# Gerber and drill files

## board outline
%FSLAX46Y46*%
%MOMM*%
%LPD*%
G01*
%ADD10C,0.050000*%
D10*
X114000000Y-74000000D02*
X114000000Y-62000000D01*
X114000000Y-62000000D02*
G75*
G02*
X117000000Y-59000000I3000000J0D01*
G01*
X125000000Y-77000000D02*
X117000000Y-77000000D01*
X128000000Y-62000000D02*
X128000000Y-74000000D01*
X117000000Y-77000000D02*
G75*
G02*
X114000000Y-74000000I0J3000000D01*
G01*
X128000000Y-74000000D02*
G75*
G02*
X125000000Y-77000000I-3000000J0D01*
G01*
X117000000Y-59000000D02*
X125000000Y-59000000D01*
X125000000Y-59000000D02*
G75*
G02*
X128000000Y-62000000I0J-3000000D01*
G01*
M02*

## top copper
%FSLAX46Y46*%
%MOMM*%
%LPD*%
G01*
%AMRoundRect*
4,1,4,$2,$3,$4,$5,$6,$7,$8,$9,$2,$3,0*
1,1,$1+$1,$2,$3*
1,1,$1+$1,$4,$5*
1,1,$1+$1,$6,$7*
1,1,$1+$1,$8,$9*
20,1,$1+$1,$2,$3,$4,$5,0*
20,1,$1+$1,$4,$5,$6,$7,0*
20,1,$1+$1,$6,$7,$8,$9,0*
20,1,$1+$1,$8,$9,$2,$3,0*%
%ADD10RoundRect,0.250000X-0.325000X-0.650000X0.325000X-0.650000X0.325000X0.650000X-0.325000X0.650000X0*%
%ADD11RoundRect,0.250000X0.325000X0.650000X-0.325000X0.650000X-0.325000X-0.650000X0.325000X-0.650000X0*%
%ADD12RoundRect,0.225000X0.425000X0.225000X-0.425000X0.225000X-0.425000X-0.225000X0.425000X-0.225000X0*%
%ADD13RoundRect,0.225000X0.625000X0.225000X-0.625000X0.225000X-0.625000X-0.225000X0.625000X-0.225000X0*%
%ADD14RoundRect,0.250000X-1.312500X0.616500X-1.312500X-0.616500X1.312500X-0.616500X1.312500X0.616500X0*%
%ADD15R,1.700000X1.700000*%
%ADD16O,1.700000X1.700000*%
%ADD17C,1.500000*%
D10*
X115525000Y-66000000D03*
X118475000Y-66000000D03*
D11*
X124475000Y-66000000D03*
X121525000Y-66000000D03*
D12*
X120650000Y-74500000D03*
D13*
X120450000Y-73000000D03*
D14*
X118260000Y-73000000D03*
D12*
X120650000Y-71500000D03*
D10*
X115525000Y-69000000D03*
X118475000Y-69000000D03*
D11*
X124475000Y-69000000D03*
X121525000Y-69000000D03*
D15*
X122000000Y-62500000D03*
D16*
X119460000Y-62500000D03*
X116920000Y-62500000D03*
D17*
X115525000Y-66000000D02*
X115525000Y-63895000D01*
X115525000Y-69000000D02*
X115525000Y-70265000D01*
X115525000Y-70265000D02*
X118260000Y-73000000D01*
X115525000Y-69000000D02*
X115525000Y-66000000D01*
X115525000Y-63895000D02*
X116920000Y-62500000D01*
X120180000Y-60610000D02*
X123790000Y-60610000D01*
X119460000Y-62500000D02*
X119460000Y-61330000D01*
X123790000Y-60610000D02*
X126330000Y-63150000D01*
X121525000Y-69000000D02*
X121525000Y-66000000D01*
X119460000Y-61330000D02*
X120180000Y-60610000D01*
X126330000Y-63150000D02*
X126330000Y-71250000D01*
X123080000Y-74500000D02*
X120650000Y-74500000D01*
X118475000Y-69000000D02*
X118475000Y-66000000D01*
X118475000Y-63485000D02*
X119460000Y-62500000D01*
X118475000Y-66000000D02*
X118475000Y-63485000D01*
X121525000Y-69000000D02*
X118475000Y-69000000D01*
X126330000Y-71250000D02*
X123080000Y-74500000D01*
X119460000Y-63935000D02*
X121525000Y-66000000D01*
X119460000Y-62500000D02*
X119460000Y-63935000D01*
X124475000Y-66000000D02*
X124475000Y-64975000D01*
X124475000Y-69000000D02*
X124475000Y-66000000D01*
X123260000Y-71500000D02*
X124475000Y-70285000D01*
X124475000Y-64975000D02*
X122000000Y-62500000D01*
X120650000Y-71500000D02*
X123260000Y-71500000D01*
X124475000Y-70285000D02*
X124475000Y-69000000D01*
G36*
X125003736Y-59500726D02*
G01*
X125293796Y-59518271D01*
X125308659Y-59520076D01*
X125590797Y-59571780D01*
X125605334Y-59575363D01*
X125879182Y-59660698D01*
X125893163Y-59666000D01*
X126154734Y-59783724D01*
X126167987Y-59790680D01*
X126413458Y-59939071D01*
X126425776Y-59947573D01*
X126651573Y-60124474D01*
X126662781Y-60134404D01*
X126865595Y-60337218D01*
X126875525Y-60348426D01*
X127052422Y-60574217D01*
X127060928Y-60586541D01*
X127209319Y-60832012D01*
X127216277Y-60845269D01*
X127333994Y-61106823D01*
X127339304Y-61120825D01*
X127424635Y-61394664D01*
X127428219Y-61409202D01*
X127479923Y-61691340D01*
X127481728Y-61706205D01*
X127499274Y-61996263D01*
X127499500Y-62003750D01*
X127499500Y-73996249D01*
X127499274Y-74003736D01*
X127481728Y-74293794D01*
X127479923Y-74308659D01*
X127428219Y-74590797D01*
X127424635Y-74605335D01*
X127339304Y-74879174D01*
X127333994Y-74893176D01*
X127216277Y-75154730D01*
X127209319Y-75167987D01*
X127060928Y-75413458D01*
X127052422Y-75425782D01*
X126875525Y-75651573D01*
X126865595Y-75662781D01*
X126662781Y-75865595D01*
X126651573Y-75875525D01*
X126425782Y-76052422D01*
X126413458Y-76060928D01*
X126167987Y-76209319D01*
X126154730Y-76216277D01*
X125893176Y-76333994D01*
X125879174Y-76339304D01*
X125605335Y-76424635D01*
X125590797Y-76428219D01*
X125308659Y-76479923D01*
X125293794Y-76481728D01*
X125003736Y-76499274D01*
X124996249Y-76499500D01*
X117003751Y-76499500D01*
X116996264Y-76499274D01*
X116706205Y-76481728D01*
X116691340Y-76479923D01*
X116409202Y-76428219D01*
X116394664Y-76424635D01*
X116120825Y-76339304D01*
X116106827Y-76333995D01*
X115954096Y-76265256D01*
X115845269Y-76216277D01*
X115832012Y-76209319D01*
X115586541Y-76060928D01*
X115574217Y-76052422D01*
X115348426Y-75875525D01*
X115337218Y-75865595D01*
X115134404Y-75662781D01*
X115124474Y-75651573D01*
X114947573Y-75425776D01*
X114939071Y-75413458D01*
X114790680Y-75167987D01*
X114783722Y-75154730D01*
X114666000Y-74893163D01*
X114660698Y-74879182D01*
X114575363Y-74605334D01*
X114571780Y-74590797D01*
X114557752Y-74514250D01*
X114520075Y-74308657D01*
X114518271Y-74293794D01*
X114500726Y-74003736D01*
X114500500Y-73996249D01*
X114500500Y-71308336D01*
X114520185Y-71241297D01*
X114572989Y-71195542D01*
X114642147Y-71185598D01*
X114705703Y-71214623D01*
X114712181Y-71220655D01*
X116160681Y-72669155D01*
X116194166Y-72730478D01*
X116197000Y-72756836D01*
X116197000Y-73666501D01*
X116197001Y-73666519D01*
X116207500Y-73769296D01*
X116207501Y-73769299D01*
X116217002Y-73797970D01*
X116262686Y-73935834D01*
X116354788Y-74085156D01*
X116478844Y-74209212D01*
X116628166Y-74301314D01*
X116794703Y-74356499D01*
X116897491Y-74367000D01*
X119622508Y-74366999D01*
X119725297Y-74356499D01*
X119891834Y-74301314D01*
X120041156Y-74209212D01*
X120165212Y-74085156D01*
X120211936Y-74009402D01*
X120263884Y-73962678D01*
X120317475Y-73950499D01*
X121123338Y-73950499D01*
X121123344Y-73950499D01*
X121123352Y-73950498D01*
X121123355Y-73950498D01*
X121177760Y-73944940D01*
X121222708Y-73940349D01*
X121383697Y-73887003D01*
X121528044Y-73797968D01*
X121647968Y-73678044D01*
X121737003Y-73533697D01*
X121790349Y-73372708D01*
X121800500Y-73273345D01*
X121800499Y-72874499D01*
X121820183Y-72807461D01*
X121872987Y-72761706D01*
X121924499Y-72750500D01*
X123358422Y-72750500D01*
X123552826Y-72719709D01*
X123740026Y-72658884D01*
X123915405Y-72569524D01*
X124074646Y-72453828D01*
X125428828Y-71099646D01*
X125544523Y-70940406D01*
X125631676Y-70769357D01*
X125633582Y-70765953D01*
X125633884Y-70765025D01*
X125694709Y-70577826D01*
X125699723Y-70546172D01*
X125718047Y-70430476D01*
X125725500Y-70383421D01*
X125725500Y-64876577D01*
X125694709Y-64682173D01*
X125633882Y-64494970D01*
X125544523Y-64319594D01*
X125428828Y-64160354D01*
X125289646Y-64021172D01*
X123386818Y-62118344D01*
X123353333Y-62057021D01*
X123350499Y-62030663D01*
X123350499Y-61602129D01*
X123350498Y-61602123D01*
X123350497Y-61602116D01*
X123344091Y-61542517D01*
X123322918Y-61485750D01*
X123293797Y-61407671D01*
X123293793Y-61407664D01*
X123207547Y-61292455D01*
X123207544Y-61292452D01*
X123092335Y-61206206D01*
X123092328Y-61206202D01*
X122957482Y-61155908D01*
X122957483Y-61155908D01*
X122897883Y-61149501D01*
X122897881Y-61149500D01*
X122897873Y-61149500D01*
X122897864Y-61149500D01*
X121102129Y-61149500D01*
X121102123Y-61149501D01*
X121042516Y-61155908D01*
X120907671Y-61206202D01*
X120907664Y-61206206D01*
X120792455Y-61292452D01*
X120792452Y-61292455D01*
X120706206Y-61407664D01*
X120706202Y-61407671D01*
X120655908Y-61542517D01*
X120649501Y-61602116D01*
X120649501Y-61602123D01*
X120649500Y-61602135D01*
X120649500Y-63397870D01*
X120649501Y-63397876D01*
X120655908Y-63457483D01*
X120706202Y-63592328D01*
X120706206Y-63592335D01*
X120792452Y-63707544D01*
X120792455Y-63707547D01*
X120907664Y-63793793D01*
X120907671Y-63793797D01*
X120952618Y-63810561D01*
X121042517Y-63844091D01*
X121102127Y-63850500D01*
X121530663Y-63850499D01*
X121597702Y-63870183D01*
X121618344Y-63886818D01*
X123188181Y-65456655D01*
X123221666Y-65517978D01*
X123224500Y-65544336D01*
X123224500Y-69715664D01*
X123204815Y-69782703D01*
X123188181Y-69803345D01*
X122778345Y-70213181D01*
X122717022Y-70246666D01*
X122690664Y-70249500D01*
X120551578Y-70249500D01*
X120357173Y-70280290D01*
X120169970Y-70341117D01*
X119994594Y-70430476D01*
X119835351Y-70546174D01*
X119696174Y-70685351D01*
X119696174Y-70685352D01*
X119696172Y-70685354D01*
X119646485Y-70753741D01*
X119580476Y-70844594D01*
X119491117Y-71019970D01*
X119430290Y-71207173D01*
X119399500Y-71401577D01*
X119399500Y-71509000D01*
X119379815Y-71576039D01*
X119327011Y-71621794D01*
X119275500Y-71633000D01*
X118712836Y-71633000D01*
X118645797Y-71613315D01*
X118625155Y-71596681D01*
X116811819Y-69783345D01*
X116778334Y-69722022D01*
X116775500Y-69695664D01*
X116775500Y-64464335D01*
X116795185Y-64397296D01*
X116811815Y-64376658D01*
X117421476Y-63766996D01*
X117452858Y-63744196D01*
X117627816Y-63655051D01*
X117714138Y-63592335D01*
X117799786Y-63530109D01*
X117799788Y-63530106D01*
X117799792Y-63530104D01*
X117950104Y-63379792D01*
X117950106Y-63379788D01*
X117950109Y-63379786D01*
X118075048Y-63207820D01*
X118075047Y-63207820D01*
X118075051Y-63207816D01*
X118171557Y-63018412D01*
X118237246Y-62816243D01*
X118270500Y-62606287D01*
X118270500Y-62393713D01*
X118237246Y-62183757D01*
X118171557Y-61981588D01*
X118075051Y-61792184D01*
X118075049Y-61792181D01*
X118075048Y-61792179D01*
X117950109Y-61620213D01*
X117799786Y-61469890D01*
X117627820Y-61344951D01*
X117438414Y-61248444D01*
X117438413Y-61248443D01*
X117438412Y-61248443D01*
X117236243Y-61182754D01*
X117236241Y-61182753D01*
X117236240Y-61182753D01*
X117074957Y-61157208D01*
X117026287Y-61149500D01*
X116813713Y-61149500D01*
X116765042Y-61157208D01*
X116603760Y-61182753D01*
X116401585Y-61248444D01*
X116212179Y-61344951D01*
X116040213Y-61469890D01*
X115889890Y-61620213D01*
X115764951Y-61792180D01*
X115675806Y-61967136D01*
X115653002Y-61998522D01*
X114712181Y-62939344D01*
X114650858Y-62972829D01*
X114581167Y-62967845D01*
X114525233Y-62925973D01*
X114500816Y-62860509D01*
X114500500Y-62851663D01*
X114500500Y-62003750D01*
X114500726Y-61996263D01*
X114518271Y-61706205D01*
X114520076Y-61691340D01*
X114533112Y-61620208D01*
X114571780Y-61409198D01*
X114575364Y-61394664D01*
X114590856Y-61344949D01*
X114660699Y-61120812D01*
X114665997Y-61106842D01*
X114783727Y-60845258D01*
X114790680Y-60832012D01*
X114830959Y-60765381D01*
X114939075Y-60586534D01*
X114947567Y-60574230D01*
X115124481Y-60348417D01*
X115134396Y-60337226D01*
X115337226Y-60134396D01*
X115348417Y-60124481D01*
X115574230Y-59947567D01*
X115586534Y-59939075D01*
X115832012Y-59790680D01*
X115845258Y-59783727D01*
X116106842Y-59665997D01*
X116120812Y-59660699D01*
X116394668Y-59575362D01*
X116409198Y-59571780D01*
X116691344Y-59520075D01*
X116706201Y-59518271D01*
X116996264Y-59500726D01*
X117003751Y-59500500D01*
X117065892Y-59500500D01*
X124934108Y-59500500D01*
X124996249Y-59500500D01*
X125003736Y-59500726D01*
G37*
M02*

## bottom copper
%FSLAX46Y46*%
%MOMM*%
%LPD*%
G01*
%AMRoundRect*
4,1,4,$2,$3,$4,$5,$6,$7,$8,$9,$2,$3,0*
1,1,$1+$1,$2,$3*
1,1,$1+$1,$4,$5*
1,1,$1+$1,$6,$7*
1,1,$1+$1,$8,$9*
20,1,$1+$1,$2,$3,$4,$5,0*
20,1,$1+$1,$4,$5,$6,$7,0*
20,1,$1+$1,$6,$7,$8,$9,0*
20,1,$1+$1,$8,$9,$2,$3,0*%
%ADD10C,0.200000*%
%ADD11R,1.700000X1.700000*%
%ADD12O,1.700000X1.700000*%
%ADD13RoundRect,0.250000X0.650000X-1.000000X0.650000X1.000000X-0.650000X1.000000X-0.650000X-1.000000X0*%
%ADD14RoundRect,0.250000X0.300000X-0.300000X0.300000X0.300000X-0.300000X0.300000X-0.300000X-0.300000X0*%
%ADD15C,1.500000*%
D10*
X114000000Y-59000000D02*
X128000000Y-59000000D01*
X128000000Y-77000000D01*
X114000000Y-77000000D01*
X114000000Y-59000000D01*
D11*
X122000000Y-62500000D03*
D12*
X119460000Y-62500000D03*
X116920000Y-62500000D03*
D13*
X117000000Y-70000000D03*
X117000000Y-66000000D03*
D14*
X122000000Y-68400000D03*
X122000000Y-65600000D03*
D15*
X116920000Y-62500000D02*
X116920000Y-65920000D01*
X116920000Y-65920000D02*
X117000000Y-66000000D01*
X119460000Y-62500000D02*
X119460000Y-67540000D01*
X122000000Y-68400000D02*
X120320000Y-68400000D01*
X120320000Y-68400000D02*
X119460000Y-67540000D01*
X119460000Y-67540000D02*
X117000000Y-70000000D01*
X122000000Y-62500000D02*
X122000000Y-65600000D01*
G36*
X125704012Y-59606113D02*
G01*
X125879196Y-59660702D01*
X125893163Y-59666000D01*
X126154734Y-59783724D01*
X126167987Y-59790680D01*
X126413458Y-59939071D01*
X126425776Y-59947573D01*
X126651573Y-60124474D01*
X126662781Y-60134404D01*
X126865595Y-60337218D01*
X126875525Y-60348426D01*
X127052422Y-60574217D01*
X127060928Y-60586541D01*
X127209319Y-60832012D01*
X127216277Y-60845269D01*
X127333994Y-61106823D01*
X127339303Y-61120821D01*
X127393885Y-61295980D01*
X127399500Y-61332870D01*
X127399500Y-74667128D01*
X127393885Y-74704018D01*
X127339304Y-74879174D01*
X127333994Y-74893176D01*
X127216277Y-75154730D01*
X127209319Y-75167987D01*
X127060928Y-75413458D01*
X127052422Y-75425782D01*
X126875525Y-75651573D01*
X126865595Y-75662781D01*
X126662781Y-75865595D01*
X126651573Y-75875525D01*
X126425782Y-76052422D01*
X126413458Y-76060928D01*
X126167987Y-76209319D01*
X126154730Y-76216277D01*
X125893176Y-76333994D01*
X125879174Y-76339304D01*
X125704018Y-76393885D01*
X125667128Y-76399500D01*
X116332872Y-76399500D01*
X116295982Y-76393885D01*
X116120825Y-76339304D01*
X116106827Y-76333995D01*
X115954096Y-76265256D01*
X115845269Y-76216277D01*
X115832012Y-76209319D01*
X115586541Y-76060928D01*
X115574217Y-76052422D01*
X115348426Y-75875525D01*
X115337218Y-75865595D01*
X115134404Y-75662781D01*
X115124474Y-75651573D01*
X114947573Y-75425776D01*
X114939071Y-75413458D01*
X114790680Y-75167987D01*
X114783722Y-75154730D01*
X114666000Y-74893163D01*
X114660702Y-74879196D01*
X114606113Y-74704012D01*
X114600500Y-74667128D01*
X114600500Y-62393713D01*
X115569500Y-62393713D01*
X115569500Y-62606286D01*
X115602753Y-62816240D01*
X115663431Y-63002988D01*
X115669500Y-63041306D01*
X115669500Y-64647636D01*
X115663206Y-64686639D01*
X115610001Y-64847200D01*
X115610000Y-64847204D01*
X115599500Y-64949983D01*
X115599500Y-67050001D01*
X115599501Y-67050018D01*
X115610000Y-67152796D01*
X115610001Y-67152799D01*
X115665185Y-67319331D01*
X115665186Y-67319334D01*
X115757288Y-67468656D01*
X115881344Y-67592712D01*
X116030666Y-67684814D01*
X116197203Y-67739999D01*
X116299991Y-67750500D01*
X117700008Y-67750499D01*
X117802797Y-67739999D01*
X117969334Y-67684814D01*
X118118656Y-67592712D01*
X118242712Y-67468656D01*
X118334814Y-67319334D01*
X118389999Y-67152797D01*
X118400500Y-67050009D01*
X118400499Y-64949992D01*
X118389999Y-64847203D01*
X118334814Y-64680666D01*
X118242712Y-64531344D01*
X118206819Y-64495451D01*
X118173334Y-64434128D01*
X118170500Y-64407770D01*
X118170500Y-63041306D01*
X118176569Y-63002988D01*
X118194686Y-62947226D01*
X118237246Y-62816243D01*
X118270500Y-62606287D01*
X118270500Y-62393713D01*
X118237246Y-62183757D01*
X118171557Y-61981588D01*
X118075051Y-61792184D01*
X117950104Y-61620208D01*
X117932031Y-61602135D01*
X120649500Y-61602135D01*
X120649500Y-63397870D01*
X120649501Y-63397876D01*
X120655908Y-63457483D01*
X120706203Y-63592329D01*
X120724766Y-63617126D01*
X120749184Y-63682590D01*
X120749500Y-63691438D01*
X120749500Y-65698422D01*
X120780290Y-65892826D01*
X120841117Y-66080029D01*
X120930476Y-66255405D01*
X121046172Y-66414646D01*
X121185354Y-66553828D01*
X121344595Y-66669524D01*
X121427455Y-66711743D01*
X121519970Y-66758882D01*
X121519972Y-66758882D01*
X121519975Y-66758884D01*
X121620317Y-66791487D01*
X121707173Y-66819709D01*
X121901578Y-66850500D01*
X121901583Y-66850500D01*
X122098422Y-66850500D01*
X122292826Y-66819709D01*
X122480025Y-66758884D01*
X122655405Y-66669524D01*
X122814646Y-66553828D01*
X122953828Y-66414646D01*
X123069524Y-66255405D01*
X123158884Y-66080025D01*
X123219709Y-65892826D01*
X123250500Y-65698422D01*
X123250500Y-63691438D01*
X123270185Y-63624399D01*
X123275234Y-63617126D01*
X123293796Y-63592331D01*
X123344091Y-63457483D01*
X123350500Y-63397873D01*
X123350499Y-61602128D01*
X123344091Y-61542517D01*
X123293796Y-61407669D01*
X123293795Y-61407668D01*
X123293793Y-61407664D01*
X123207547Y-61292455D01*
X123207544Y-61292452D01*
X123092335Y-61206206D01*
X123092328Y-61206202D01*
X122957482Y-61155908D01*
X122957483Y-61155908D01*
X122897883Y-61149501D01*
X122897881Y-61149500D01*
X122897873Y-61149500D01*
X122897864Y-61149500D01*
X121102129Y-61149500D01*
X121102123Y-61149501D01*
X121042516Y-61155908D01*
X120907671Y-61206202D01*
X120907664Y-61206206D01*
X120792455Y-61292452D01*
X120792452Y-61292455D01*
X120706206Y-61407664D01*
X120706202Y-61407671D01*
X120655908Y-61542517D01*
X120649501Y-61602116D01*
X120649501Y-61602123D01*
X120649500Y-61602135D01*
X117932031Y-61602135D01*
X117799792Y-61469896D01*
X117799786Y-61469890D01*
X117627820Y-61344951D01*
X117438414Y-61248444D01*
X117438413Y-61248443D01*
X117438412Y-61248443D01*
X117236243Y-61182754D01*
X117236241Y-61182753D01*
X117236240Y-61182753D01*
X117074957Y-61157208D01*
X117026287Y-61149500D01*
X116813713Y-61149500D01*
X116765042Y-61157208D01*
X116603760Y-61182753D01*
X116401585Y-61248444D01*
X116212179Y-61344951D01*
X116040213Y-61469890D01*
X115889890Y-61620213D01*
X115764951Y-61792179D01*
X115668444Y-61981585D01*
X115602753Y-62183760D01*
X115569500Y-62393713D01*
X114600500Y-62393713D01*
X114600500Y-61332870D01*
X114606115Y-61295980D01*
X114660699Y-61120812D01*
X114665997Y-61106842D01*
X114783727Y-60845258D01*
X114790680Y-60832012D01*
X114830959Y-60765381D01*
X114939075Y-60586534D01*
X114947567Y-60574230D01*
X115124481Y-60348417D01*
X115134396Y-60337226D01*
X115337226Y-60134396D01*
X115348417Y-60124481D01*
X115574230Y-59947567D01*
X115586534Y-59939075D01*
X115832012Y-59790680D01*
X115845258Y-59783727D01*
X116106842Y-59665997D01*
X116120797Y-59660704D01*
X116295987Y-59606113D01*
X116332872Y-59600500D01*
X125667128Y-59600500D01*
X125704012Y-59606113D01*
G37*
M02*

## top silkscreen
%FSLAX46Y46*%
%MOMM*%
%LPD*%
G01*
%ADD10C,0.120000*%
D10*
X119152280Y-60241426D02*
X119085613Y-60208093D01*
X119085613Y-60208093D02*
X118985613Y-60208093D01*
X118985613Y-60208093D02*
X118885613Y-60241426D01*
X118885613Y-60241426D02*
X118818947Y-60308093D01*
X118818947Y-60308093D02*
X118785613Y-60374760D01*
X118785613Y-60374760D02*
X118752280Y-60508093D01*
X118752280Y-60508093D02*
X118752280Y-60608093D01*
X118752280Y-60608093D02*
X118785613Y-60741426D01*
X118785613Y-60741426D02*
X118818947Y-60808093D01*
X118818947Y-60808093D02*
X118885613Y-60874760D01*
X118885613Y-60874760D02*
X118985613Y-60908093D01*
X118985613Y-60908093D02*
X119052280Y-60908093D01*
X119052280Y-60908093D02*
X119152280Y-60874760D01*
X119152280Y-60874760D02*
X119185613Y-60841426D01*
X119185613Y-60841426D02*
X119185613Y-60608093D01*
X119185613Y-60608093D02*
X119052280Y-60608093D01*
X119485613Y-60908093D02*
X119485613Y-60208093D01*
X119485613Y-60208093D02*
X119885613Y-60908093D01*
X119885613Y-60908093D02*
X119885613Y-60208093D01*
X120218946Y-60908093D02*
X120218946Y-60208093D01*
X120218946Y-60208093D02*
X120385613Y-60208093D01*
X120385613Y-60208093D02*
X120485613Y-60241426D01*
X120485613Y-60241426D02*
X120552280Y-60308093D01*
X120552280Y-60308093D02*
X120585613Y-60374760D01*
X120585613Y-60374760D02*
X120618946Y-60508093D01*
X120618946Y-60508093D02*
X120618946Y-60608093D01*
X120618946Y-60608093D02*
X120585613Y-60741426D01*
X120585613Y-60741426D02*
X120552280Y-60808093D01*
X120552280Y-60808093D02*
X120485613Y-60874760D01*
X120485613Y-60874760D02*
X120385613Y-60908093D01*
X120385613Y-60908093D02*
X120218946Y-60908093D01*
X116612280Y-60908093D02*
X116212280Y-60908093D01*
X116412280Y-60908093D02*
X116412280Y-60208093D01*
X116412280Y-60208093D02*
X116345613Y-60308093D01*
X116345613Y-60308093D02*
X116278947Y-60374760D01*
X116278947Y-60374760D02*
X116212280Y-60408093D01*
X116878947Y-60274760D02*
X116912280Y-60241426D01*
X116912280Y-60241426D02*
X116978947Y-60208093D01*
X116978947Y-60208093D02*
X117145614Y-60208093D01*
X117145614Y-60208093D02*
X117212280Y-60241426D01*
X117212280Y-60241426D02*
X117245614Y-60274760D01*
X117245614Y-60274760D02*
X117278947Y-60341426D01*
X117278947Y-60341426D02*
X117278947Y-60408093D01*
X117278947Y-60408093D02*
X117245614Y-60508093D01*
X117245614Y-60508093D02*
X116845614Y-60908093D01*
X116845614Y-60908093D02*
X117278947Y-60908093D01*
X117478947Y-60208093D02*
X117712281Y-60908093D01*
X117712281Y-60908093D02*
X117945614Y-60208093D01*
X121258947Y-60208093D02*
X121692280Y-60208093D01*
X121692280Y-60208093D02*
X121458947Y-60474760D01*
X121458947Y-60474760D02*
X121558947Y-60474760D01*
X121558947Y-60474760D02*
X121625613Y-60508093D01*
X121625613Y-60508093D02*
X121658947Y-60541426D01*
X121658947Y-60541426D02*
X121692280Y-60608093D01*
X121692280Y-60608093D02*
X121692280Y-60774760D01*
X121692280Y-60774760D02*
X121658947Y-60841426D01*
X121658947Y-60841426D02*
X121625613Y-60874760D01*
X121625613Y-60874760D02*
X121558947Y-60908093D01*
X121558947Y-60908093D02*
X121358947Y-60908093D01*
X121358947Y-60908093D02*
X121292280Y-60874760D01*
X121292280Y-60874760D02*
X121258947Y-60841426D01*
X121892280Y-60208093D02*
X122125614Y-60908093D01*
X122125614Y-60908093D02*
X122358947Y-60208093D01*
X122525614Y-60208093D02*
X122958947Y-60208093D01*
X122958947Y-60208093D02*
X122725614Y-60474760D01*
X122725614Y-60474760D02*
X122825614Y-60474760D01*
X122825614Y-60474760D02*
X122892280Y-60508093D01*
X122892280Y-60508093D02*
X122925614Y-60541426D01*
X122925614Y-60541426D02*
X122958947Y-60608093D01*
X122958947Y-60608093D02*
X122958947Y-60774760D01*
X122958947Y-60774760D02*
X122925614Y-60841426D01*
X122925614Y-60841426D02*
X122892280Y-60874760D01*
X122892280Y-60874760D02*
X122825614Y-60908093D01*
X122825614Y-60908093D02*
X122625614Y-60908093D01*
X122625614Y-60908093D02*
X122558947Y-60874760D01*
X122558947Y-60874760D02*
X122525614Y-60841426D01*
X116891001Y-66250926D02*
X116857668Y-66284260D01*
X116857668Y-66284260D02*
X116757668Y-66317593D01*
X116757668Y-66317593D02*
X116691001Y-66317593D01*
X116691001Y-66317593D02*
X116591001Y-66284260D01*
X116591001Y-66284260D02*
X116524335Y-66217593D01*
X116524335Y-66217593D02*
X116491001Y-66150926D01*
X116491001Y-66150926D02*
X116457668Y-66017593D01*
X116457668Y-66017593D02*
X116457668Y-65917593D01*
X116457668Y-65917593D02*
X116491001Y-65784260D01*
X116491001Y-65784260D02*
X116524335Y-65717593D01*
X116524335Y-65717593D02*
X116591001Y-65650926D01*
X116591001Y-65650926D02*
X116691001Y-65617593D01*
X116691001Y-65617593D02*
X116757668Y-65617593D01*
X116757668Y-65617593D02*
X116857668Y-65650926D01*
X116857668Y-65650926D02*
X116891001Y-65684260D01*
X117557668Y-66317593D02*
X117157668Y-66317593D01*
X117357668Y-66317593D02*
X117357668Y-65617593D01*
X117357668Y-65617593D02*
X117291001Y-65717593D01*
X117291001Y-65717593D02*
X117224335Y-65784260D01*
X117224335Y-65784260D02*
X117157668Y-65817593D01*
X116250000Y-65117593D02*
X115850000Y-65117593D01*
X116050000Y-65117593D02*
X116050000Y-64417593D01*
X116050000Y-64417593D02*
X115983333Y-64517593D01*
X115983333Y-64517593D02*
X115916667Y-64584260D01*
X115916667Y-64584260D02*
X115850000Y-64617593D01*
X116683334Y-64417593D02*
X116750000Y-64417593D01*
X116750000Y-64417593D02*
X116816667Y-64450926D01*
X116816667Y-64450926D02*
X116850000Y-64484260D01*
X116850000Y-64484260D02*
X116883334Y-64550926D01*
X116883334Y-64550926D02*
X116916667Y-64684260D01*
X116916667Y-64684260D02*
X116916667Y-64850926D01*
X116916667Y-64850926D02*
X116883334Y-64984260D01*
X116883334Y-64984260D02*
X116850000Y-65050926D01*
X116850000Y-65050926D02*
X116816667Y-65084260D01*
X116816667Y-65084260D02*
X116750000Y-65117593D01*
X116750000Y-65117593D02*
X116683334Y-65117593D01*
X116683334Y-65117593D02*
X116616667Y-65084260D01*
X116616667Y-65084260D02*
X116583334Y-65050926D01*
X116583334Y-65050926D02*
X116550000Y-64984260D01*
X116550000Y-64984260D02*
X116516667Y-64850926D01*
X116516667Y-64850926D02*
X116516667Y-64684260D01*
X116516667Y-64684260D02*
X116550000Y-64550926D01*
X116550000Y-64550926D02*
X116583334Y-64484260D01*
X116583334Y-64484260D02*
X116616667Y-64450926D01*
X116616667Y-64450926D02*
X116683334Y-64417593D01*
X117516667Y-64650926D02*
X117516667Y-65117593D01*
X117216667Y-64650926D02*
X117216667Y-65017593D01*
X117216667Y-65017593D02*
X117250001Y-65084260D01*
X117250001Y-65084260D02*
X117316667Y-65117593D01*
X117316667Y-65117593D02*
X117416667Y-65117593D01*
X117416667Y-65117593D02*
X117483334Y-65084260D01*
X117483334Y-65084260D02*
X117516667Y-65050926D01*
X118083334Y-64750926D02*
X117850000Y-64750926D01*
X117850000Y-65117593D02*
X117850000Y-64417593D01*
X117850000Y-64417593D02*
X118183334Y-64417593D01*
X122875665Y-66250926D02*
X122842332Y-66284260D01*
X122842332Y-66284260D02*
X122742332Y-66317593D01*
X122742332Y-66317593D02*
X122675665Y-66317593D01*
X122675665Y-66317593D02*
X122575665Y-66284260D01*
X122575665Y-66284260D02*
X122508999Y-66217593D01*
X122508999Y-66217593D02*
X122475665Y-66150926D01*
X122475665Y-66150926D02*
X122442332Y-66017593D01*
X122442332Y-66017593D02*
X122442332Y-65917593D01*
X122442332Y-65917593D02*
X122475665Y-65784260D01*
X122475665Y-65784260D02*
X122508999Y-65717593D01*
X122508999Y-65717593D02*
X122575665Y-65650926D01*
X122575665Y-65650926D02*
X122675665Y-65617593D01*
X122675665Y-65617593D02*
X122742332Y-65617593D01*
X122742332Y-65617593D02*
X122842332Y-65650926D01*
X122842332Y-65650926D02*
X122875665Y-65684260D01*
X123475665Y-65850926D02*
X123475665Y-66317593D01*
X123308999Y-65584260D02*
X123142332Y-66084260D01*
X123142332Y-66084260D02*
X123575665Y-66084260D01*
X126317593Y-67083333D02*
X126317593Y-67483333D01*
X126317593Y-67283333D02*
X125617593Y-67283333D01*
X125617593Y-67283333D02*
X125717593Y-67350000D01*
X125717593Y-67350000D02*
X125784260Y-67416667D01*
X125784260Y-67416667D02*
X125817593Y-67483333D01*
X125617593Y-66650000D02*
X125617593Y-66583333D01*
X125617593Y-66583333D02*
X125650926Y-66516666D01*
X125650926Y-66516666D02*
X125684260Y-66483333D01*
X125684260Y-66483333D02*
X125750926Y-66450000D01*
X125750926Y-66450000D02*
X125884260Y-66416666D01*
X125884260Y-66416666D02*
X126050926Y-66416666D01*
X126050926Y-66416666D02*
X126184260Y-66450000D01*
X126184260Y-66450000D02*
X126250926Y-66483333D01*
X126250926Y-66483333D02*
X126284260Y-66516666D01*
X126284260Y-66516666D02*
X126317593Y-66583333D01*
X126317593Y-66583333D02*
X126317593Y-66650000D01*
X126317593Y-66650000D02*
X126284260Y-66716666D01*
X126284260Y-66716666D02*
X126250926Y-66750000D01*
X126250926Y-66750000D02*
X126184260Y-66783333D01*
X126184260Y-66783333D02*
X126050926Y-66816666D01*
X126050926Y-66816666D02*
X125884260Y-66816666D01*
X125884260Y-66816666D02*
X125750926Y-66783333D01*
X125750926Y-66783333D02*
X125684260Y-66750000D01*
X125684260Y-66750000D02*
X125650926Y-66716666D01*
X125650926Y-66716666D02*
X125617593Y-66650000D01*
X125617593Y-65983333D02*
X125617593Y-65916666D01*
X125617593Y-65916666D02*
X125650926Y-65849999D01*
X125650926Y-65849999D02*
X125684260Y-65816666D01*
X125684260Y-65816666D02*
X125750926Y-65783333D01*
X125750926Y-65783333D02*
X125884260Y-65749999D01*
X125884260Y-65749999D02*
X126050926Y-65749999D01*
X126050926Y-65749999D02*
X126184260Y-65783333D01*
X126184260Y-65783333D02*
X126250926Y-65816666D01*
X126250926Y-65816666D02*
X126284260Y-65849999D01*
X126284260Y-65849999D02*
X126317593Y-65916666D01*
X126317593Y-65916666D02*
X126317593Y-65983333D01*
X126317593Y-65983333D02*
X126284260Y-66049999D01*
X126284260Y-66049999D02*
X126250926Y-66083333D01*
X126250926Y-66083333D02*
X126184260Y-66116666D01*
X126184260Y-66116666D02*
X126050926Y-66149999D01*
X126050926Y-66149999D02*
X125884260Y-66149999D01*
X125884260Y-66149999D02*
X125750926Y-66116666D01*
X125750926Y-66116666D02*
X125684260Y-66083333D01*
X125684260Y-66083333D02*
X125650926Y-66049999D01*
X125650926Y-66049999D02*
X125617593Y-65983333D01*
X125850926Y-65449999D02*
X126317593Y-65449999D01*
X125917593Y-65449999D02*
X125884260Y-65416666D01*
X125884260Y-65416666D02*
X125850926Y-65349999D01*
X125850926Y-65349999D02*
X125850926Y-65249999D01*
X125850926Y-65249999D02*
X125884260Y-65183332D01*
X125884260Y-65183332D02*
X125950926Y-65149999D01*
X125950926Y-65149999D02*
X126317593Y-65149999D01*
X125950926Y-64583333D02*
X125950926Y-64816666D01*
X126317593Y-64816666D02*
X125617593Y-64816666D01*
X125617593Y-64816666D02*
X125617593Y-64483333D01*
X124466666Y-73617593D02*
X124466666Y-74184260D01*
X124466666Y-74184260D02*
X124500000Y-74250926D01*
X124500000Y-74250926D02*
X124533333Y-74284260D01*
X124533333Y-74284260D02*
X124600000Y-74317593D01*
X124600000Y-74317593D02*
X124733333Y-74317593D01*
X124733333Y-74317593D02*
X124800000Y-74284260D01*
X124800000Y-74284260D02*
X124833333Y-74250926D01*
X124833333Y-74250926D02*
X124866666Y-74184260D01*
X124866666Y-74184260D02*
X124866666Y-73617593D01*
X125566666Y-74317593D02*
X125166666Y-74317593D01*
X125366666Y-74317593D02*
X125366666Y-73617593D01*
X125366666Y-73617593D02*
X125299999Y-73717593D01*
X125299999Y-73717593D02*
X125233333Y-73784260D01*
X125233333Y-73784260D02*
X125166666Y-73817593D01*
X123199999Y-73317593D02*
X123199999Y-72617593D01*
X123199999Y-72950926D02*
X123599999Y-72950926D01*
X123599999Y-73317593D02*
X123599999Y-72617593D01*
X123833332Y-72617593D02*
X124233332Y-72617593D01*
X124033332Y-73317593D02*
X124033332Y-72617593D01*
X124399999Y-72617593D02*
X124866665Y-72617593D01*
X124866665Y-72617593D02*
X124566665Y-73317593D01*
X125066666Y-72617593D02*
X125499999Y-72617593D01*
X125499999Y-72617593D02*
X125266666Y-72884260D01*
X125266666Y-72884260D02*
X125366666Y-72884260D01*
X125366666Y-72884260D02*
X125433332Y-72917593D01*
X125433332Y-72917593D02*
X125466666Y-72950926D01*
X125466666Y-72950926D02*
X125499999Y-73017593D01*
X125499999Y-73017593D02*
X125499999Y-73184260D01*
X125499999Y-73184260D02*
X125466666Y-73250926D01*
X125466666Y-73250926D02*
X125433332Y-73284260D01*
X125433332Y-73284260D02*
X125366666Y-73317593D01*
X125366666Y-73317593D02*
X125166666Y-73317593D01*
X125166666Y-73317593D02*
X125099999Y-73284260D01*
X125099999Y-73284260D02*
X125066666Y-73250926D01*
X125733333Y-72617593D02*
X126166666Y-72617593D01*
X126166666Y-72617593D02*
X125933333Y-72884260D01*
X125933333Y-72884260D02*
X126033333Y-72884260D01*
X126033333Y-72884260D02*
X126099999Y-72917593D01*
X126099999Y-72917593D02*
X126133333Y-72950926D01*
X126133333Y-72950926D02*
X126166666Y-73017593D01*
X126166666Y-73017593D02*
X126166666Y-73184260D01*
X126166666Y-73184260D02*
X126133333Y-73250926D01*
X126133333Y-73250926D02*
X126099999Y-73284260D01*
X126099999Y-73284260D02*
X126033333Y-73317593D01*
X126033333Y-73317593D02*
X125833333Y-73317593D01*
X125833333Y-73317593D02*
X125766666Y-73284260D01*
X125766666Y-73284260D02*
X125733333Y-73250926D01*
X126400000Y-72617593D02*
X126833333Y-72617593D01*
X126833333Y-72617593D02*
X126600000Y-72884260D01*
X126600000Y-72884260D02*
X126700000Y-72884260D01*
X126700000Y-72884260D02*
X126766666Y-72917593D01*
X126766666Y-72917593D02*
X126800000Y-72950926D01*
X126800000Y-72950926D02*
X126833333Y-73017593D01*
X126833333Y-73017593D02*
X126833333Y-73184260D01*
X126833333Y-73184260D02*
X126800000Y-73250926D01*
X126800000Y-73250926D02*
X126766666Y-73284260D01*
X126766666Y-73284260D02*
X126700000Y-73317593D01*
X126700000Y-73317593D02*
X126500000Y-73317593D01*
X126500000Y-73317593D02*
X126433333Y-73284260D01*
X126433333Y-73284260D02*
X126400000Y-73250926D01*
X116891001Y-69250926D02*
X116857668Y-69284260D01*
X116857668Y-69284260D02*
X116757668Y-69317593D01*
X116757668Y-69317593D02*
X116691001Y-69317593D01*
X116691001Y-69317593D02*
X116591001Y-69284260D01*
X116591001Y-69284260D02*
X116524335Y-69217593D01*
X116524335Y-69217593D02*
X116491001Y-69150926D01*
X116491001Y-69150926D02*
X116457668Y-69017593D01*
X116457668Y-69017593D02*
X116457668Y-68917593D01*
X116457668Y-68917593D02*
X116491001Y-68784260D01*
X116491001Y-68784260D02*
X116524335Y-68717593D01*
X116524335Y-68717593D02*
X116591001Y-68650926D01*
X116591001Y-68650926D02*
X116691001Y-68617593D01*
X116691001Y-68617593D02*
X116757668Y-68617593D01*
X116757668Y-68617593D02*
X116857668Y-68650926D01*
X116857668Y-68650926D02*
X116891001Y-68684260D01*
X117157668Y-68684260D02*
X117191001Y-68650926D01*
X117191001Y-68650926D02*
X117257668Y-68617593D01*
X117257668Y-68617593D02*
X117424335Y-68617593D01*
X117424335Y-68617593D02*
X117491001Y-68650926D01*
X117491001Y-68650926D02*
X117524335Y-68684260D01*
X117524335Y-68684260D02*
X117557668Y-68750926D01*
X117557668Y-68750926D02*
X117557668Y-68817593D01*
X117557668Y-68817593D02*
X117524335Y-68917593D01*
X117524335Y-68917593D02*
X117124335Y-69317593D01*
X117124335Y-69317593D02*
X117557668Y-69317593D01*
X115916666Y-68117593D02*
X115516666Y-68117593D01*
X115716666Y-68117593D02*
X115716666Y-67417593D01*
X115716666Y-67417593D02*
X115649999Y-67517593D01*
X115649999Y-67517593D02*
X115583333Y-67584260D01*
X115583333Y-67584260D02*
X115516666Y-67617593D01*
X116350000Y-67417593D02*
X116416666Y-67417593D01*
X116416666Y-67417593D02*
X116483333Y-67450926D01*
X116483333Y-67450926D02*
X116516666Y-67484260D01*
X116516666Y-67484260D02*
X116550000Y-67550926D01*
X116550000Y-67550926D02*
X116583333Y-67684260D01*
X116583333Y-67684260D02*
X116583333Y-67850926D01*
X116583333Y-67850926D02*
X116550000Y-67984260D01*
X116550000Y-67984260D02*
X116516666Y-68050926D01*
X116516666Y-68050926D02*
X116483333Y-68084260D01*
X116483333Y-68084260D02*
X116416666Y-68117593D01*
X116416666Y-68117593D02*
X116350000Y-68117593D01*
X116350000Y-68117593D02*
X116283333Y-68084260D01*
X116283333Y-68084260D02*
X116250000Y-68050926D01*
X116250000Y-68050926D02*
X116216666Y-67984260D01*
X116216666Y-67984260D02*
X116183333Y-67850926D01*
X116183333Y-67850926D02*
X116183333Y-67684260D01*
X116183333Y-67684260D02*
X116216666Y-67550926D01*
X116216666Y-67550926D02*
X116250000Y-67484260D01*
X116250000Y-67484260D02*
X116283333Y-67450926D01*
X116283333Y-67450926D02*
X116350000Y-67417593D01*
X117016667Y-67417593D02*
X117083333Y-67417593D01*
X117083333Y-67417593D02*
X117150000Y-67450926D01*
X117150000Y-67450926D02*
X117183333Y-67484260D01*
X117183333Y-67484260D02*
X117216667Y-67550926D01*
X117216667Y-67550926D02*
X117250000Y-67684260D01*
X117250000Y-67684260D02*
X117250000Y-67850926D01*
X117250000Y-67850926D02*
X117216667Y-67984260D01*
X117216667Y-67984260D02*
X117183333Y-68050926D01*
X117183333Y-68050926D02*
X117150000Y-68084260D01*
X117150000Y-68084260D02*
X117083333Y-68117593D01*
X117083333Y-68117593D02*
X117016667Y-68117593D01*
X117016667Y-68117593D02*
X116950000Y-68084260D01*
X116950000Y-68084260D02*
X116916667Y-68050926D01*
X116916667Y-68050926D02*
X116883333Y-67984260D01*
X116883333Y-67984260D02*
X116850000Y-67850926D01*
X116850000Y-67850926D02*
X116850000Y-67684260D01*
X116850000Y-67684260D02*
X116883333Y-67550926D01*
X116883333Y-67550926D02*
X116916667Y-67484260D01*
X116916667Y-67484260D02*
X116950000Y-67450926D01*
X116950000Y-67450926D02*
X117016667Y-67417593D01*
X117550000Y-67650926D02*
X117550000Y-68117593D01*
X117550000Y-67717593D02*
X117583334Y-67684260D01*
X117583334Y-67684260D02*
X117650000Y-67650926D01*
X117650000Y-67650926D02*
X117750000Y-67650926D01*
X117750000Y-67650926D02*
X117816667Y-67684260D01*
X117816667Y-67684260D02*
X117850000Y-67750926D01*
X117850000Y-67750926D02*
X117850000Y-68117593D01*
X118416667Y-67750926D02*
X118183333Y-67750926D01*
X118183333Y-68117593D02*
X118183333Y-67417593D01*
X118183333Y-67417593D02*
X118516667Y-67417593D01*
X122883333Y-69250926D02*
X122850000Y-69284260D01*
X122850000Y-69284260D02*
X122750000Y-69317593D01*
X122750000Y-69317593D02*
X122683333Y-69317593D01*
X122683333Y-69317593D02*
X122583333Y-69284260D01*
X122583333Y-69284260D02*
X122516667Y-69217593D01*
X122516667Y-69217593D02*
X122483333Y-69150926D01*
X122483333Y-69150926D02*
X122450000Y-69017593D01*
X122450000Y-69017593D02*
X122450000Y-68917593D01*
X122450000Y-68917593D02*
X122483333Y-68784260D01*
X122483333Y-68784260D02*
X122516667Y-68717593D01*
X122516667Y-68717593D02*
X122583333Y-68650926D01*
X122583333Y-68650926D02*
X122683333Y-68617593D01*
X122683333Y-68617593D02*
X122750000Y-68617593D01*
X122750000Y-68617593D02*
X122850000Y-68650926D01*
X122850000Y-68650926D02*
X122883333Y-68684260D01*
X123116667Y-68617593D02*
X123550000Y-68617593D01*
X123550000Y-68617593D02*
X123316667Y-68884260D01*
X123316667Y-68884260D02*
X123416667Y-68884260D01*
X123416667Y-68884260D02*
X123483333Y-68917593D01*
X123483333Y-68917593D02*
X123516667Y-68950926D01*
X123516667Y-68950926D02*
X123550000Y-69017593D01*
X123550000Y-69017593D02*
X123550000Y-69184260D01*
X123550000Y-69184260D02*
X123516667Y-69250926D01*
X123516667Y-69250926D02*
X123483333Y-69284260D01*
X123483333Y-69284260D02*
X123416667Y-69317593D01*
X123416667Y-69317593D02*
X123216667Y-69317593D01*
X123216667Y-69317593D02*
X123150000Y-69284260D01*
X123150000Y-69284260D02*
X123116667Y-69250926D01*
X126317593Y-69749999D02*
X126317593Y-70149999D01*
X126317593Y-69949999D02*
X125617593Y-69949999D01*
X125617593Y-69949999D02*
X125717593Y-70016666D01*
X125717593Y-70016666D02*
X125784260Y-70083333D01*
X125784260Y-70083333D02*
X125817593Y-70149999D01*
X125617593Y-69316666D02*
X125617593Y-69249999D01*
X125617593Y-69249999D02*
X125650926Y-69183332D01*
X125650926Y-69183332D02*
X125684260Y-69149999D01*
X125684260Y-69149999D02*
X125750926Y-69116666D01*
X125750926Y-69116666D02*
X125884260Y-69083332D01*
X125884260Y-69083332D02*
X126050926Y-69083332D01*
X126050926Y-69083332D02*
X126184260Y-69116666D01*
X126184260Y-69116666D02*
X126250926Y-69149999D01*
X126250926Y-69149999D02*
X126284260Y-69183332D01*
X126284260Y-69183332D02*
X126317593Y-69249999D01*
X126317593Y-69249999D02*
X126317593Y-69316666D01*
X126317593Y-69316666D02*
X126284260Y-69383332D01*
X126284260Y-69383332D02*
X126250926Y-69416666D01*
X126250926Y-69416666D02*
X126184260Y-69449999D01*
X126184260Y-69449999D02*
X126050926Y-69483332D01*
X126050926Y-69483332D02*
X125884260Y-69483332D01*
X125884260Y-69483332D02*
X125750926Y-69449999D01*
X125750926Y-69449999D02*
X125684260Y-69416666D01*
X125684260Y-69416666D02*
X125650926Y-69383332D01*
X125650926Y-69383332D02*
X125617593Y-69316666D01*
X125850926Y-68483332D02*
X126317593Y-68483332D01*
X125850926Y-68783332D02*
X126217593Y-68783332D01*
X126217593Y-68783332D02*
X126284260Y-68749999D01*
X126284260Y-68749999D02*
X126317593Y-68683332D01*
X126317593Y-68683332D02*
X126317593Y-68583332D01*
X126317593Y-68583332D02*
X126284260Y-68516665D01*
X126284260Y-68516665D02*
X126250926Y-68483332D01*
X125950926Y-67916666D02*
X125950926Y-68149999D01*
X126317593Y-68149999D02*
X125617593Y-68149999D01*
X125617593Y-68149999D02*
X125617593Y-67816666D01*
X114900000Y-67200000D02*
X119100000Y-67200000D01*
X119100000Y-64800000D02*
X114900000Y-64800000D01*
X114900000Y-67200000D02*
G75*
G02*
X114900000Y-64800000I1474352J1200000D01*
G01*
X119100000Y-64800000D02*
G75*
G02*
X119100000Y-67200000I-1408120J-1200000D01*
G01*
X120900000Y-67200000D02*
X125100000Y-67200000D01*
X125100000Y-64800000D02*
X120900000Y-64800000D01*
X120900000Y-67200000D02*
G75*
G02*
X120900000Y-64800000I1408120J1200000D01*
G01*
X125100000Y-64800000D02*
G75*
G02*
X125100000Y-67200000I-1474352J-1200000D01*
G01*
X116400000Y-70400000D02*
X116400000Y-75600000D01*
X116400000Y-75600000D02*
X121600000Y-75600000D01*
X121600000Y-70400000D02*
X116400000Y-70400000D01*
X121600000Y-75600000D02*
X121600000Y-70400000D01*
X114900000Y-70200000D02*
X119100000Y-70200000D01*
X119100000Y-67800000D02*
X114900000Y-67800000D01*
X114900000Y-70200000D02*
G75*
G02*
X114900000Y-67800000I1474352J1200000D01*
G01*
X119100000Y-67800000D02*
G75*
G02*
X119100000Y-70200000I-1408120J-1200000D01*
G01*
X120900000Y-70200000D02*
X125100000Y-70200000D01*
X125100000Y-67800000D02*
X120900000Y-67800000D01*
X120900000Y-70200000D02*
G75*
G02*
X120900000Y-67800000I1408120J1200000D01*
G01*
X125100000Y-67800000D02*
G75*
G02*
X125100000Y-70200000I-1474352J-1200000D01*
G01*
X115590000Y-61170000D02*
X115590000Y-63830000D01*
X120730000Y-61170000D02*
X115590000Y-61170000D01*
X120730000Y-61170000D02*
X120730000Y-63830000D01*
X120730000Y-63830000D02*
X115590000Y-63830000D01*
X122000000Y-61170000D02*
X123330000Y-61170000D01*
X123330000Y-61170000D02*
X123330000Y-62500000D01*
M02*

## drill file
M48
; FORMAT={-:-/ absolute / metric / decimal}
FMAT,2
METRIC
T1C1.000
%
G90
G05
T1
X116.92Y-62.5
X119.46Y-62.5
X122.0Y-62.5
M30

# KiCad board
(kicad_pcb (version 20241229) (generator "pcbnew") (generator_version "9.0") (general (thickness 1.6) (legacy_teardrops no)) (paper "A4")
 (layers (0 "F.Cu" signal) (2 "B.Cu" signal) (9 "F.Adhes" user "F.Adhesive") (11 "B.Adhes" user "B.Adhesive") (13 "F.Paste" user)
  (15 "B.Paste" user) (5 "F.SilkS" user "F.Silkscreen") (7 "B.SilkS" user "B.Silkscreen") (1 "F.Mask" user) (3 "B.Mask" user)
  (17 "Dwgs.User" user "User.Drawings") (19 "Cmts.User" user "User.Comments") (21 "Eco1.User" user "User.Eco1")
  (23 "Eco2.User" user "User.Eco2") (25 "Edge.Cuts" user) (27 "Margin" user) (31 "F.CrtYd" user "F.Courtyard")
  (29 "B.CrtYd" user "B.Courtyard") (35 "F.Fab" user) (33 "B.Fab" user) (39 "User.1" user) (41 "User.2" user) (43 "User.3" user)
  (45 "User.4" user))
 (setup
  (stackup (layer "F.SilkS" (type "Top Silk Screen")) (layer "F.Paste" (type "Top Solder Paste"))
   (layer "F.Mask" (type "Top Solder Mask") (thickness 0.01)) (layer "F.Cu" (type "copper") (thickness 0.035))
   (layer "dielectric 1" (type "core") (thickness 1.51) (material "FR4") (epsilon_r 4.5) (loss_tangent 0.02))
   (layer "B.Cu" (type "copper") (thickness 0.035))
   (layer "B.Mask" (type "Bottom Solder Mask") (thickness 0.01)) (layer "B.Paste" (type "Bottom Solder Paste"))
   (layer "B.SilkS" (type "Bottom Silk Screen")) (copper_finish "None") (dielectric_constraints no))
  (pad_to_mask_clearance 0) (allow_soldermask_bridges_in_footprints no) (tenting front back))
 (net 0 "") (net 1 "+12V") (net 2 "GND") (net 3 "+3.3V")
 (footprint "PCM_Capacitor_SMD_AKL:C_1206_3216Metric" (layer "F.Cu") (at 117 66)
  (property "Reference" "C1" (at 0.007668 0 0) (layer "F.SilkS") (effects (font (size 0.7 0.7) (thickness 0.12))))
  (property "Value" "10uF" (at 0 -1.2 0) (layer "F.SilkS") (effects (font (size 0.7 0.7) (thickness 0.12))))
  (fp_line (start -2.1 1.2) (end 2.1 1.2) (stroke (width 0.12) (type solid)) (layer "F.SilkS"))
  (fp_line (start 2.1 -1.2) (end -2.1 -1.2) (stroke (width 0.12) (type solid)) (layer "F.SilkS"))
  (fp_arc (start -2.1 1.2) (mid -2.526625 0) (end -2.1 -1.2) (stroke (width 0.12) (type solid)) (layer "F.SilkS"))
  (fp_arc (start 2.1 -1.2) (mid 2.541962 0) (end 2.1 1.2) (stroke (width 0.12) (type solid)) (layer "F.SilkS"))
  (pad "1" smd roundrect (at -1.475 0) (size 1.15 1.8) (layers "F.Cu" "F.Mask" "F.Paste") (roundrect_rratio 0.217391) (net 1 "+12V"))
  (pad "2" smd roundrect (at 1.475 0) (size 1.15 1.8) (layers "F.Cu" "F.Mask" "F.Paste") (roundrect_rratio 0.217391) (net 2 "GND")))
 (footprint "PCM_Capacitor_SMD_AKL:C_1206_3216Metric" (layer "F.Cu") (at 123 66 180)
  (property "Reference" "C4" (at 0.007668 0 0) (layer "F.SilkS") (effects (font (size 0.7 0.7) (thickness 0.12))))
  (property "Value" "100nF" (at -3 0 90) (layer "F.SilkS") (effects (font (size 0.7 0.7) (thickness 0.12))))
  (fp_line (start 2.1 -1.2) (end -2.1 -1.2) (stroke (width 0.12) (type solid)) (layer "F.SilkS"))
  (fp_line (start -2.1 1.2) (end 2.1 1.2) (stroke (width 0.12) (type solid)) (layer "F.SilkS"))
  (fp_arc (start 2.1 -1.2) (mid 2.541962 0) (end 2.1 1.2) (stroke (width 0.12) (type solid)) (layer "F.SilkS"))
  (fp_arc (start -2.1 1.2) (mid -2.526625 0) (end -2.1 -1.2) (stroke (width 0.12) (type solid)) (layer "F.SilkS"))
  (pad "1" smd roundrect (at -1.475 0 180) (size 1.15 1.8) (layers "F.Cu" "F.Mask" "F.Paste") (roundrect_rratio 0.217391) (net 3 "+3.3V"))
  (pad "2" smd roundrect (at 1.475 0 180) (size 1.15 1.8) (layers "F.Cu" "F.Mask" "F.Paste") (roundrect_rratio 0.217391) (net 2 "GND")))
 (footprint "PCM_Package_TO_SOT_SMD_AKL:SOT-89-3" (layer "F.Cu") (at 119 73 180)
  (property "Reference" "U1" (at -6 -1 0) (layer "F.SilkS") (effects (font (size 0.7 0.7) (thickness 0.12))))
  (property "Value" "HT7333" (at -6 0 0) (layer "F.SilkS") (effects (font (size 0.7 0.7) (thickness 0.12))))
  (fp_line (start 2.6 2.6) (end 2.6 -2.6) (stroke (width 0.12) (type solid)) (layer "F.SilkS"))
  (fp_line (start 2.6 -2.6) (end -2.6 -2.6) (stroke (width 0.12) (type solid)) (layer "F.SilkS"))
  (fp_line (start -2.6 2.6) (end 2.6 2.6) (stroke (width 0.12) (type solid)) (layer "F.SilkS"))
  (fp_line (start -2.6 -2.6) (end -2.6 2.6) (stroke (width 0.12) (type solid)) (layer "F.SilkS"))
  (pad "1" smd roundrect (at -1.65 -1.5 180) (size 1.3 0.9) (layers "F.Cu" "F.Mask" "F.Paste") (roundrect_rratio 0.25) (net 2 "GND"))
  (pad "2" smd roundrect (at -1.45 0 180) (size 1.7 0.9) (layers "F.Cu" "F.Mask" "F.Paste") (roundrect_rratio 0.25) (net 1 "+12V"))
  (pad "2" smd roundrect (at 0.74 0 270) (size 1.733 3.125) (layers "F.Cu" "F.Mask" "F.Paste") (roundrect_rratio 0.1442585113)
   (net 1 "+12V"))
  (pad "3" smd roundrect (at -1.65 1.5 180) (size 1.3 0.9) (layers "F.Cu" "F.Mask" "F.Paste") (roundrect_rratio 0.25) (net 3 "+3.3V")))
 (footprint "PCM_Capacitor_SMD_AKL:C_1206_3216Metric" (layer "F.Cu") (at 117 69)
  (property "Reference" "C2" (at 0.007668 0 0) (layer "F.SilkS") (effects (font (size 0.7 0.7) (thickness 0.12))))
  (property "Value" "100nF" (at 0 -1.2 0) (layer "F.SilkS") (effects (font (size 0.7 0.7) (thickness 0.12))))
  (fp_line (start -2.1 1.2) (end 2.1 1.2) (stroke (width 0.12) (type solid)) (layer "F.SilkS"))
  (fp_line (start 2.1 -1.2) (end -2.1 -1.2) (stroke (width 0.12) (type solid)) (layer "F.SilkS"))
  (fp_arc (start -2.1 1.2) (mid -2.526625 0) (end -2.1 -1.2) (stroke (width 0.12) (type solid)) (layer "F.SilkS"))
  (fp_arc (start 2.1 -1.2) (mid 2.541962 0) (end 2.1 1.2) (stroke (width 0.12) (type solid)) (layer "F.SilkS"))
  (pad "1" smd roundrect (at -1.475 0) (size 1.15 1.8) (layers "F.Cu" "F.Mask" "F.Paste") (roundrect_rratio 0.217391) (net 1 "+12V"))
  (pad "2" smd roundrect (at 1.475 0) (size 1.15 1.8) (layers "F.Cu" "F.Mask" "F.Paste") (roundrect_rratio 0.217391) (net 2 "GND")))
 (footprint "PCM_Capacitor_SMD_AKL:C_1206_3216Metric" (layer "F.Cu") (at 123 69 180)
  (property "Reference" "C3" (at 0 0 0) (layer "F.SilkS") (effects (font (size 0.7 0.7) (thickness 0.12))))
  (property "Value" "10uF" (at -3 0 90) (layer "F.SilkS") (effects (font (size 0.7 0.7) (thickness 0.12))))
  (fp_line (start 2.1 -1.2) (end -2.1 -1.2) (stroke (width 0.12) (type solid)) (layer "F.SilkS"))
  (fp_line (start -2.1 1.2) (end 2.1 1.2) (stroke (width 0.12) (type solid)) (layer "F.SilkS"))
  (fp_arc (start 2.1 -1.2) (mid 2.541962 0) (end 2.1 1.2) (stroke (width 0.12) (type solid)) (layer "F.SilkS"))
  (fp_arc (start -2.1 1.2) (mid -2.526625 0) (end -2.1 -1.2) (stroke (width 0.12) (type solid)) (layer "F.SilkS"))
  (pad "1" smd roundrect (at -1.475 0 180) (size 1.15 1.8) (layers "F.Cu" "F.Mask" "F.Paste") (roundrect_rratio 0.217391) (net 3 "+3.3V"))
  (pad "2" smd roundrect (at 1.475 0 180) (size 1.15 1.8) (layers "F.Cu" "F.Mask" "F.Paste") (roundrect_rratio 0.217391) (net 2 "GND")))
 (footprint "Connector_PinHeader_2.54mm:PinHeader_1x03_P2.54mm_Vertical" (layer "F.Cu") (at 122 62.5 -90)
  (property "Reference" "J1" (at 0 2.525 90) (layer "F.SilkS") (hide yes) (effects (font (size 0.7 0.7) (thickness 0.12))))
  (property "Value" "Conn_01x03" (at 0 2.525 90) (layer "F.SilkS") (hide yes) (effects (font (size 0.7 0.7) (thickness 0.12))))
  (fp_line (start -1.33 6.41) (end 1.33 6.41) (stroke (width 0.12) (type solid)) (layer "F.SilkS"))
  (fp_line (start -1.33 1.27) (end -1.33 6.41) (stroke (width 0.12) (type solid)) (layer "F.SilkS"))
  (fp_line (start -1.33 1.27) (end 1.33 1.27) (stroke (width 0.12) (type solid)) (layer "F.SilkS"))
  (fp_line (start 1.33 1.27) (end 1.33 6.41) (stroke (width 0.12) (type solid)) (layer "F.SilkS"))
  (fp_line (start -1.33 0) (end -1.33 -1.33) (stroke (width 0.12) (type solid)) (layer "F.SilkS"))
  (fp_line (start -1.33 -1.33) (end 0 -1.33) (stroke (width 0.12) (type solid)) (layer "F.SilkS"))
  (pad "1" thru_hole rect (at 0 0 270) (size 1.7 1.7) (drill 1) (layers "*.Cu" "*.Mask") (remove_unused_layers no) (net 3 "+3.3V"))
  (pad "2" thru_hole oval (at 0 2.54 270) (size 1.7 1.7) (drill 1) (layers "*.Cu" "*.Mask") (remove_unused_layers no) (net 2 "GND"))
  (pad "3" thru_hole oval (at 0 5.08 270) (size 1.7 1.7) (drill 1) (layers "*.Cu" "*.Mask") (remove_unused_layers no) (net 1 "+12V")))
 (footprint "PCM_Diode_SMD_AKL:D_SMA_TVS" (layer "B.Cu") (at 117 68 90)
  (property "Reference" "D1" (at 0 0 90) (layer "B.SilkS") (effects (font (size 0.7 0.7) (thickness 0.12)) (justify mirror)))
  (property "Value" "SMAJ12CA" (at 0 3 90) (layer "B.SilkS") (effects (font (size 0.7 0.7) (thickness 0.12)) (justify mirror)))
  (pad "1" smd roundrect (at -2 0 90) (size 2.5 1.8) (layers "B.Cu" "B.Mask" "B.Paste") (roundrect_rratio 0.1388888889) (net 2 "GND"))
  (pad "2" smd roundrect (at 2 0 90) (size 2.5 1.8) (layers "B.Cu" "B.Mask" "B.Paste") (roundrect_rratio 0.1388888889) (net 1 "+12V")))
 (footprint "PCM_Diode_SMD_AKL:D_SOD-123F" (layer "B.Cu") (at 122 67 90)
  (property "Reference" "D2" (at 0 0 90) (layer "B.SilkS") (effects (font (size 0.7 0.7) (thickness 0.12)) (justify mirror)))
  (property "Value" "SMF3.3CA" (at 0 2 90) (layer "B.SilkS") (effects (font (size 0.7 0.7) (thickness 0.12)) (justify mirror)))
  (pad "1" smd roundrect (at -1.4 0 90) (size 1.1 1.1) (layers "B.Cu" "B.Mask" "B.Paste") (roundrect_rratio 0.2272727273) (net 2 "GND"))
  (pad "2" smd roundrect (at 1.4 0 90) (size 1.1 1.1) (layers "B.Cu" "B.Mask" "B.Paste") (roundrect_rratio 0.2272727273) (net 3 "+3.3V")))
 (gr_rect (start 114 59) (end 128 77) (stroke (width 0.2) (type default)) (fill no) (layer "B.Cu"))
 (gr_line (start 114 74) (end 114 62) (stroke (width 0.05) (type default)) (layer "Edge.Cuts"))
 (gr_arc (start 114 62) (mid 114.87868 59.87868) (end 117 59) (stroke (width 0.05) (type default)) (layer "Edge.Cuts"))
 (gr_line (start 125 77) (end 117 77) (stroke (width 0.05) (type default)) (layer "Edge.Cuts"))
 (gr_line (start 128 62) (end 128 74) (stroke (width 0.05) (type default)) (layer "Edge.Cuts"))
 (gr_arc (start 117 77) (mid 114.87868 76.12132) (end 114 74) (stroke (width 0.05) (type default)) (layer "Edge.Cuts"))
 (gr_arc (start 128 74) (mid 127.12132 76.12132) (end 125 77) (stroke (width 0.05) (type default)) (layer "Edge.Cuts"))
 (gr_line (start 117 59) (end 125 59) (stroke (width 0.05) (type default)) (layer "Edge.Cuts"))
 (gr_arc (start 125 59) (mid 127.12132 59.87868) (end 128 62) (stroke (width 0.05) (type default)) (layer "Edge.Cuts"))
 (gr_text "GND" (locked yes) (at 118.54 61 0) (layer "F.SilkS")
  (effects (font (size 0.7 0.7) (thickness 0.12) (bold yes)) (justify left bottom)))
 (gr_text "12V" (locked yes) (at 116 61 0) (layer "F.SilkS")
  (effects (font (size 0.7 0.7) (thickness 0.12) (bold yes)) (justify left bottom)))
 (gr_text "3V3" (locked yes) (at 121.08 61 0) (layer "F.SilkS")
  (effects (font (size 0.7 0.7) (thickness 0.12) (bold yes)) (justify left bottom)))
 (segment (start 115.525 66) (end 115.525 63.895) (width 1.5) (layer "F.Cu") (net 1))
 (segment (start 115.525 69) (end 115.525 70.265) (width 1.5) (layer "F.Cu") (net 1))
 (segment (start 115.525 70.265) (end 118.26 73) (width 1.5) (layer "F.Cu") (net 1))
 (segment (start 115.525 69) (end 115.525 66) (width 1.5) (layer "F.Cu") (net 1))
 (segment (start 115.525 63.895) (end 116.92 62.5) (width 1.5) (layer "F.Cu") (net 1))
 (segment (start 116.92 62.5) (end 116.92 65.92) (width 1.5) (layer "B.Cu") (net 1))
 (segment (start 116.92 65.92) (end 117 66) (width 1.5) (layer "B.Cu") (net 1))
 (segment (start 120.18 60.61) (end 123.79 60.61) (width 1.5) (layer "F.Cu") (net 2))
 (segment (start 119.46 62.5) (end 119.46 61.33) (width 1.5) (layer "F.Cu") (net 2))
 (segment (start 123.79 60.61) (end 126.33 63.15) (width 1.5) (layer "F.Cu") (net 2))
 (segment (start 121.525 69) (end 121.525 66) (width 1.5) (layer "F.Cu") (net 2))
 (segment (start 119.46 61.33) (end 120.18 60.61) (width 1.5) (layer "F.Cu") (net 2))
 (segment (start 126.33 63.15) (end 126.33 71.25) (width 1.5) (layer "F.Cu") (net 2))
 (segment (start 123.08 74.5) (end 120.65 74.5) (width 1.5) (layer "F.Cu") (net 2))
 (segment (start 118.475 69) (end 118.475 66) (width 1.5) (layer "F.Cu") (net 2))
 (segment (start 118.475 63.485) (end 119.46 62.5) (width 1.5) (layer "F.Cu") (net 2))
 (segment (start 118.475 66) (end 118.475 63.485) (width 1.5) (layer "F.Cu") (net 2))
 (segment (start 121.525 69) (end 118.475 69) (width 1.5) (layer "F.Cu") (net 2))
 (segment (start 126.33 71.25) (end 123.08 74.5) (width 1.5) (layer "F.Cu") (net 2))
 (segment (start 119.46 63.935) (end 121.525 66) (width 1.5) (layer "F.Cu") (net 2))
 (segment (start 119.46 62.5) (end 119.46 63.935) (width 1.5) (layer "F.Cu") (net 2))
 (segment (start 119.46 62.5) (end 119.46 67.54) (width 1.5) (layer "B.Cu") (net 2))
 (segment (start 122 68.4) (end 120.32 68.4) (width 1.5) (layer "B.Cu") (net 2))
 (segment (start 120.32 68.4) (end 119.46 67.54) (width 1.5) (layer "B.Cu") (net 2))
 (segment (start 119.46 67.54) (end 117 70) (width 1.5) (layer "B.Cu") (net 2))
 (segment (start 124.475 66) (end 124.475 64.975) (width 1.5) (layer "F.Cu") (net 3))
 (segment (start 124.475 69) (end 124.475 66) (width 1.5) (layer "F.Cu") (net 3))
 (segment (start 123.26 71.5) (end 124.475 70.285) (width 1.5) (layer "F.Cu") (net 3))
 (segment (start 124.475 64.975) (end 122 62.5) (width 1.5) (layer "F.Cu") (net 3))
 (segment (start 120.65 71.5) (end 123.26 71.5) (width 1.5) (layer "F.Cu") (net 3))
 (segment (start 124.475 70.285) (end 124.475 69) (width 1.5) (layer "F.Cu") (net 3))
 (segment (start 122 62.5) (end 122 65.6) (width 1.5) (layer "B.Cu") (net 3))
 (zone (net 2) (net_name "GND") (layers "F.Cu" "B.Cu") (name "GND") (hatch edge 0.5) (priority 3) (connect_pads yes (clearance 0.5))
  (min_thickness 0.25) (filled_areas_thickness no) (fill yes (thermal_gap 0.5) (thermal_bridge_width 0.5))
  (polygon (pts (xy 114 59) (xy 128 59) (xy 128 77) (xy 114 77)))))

